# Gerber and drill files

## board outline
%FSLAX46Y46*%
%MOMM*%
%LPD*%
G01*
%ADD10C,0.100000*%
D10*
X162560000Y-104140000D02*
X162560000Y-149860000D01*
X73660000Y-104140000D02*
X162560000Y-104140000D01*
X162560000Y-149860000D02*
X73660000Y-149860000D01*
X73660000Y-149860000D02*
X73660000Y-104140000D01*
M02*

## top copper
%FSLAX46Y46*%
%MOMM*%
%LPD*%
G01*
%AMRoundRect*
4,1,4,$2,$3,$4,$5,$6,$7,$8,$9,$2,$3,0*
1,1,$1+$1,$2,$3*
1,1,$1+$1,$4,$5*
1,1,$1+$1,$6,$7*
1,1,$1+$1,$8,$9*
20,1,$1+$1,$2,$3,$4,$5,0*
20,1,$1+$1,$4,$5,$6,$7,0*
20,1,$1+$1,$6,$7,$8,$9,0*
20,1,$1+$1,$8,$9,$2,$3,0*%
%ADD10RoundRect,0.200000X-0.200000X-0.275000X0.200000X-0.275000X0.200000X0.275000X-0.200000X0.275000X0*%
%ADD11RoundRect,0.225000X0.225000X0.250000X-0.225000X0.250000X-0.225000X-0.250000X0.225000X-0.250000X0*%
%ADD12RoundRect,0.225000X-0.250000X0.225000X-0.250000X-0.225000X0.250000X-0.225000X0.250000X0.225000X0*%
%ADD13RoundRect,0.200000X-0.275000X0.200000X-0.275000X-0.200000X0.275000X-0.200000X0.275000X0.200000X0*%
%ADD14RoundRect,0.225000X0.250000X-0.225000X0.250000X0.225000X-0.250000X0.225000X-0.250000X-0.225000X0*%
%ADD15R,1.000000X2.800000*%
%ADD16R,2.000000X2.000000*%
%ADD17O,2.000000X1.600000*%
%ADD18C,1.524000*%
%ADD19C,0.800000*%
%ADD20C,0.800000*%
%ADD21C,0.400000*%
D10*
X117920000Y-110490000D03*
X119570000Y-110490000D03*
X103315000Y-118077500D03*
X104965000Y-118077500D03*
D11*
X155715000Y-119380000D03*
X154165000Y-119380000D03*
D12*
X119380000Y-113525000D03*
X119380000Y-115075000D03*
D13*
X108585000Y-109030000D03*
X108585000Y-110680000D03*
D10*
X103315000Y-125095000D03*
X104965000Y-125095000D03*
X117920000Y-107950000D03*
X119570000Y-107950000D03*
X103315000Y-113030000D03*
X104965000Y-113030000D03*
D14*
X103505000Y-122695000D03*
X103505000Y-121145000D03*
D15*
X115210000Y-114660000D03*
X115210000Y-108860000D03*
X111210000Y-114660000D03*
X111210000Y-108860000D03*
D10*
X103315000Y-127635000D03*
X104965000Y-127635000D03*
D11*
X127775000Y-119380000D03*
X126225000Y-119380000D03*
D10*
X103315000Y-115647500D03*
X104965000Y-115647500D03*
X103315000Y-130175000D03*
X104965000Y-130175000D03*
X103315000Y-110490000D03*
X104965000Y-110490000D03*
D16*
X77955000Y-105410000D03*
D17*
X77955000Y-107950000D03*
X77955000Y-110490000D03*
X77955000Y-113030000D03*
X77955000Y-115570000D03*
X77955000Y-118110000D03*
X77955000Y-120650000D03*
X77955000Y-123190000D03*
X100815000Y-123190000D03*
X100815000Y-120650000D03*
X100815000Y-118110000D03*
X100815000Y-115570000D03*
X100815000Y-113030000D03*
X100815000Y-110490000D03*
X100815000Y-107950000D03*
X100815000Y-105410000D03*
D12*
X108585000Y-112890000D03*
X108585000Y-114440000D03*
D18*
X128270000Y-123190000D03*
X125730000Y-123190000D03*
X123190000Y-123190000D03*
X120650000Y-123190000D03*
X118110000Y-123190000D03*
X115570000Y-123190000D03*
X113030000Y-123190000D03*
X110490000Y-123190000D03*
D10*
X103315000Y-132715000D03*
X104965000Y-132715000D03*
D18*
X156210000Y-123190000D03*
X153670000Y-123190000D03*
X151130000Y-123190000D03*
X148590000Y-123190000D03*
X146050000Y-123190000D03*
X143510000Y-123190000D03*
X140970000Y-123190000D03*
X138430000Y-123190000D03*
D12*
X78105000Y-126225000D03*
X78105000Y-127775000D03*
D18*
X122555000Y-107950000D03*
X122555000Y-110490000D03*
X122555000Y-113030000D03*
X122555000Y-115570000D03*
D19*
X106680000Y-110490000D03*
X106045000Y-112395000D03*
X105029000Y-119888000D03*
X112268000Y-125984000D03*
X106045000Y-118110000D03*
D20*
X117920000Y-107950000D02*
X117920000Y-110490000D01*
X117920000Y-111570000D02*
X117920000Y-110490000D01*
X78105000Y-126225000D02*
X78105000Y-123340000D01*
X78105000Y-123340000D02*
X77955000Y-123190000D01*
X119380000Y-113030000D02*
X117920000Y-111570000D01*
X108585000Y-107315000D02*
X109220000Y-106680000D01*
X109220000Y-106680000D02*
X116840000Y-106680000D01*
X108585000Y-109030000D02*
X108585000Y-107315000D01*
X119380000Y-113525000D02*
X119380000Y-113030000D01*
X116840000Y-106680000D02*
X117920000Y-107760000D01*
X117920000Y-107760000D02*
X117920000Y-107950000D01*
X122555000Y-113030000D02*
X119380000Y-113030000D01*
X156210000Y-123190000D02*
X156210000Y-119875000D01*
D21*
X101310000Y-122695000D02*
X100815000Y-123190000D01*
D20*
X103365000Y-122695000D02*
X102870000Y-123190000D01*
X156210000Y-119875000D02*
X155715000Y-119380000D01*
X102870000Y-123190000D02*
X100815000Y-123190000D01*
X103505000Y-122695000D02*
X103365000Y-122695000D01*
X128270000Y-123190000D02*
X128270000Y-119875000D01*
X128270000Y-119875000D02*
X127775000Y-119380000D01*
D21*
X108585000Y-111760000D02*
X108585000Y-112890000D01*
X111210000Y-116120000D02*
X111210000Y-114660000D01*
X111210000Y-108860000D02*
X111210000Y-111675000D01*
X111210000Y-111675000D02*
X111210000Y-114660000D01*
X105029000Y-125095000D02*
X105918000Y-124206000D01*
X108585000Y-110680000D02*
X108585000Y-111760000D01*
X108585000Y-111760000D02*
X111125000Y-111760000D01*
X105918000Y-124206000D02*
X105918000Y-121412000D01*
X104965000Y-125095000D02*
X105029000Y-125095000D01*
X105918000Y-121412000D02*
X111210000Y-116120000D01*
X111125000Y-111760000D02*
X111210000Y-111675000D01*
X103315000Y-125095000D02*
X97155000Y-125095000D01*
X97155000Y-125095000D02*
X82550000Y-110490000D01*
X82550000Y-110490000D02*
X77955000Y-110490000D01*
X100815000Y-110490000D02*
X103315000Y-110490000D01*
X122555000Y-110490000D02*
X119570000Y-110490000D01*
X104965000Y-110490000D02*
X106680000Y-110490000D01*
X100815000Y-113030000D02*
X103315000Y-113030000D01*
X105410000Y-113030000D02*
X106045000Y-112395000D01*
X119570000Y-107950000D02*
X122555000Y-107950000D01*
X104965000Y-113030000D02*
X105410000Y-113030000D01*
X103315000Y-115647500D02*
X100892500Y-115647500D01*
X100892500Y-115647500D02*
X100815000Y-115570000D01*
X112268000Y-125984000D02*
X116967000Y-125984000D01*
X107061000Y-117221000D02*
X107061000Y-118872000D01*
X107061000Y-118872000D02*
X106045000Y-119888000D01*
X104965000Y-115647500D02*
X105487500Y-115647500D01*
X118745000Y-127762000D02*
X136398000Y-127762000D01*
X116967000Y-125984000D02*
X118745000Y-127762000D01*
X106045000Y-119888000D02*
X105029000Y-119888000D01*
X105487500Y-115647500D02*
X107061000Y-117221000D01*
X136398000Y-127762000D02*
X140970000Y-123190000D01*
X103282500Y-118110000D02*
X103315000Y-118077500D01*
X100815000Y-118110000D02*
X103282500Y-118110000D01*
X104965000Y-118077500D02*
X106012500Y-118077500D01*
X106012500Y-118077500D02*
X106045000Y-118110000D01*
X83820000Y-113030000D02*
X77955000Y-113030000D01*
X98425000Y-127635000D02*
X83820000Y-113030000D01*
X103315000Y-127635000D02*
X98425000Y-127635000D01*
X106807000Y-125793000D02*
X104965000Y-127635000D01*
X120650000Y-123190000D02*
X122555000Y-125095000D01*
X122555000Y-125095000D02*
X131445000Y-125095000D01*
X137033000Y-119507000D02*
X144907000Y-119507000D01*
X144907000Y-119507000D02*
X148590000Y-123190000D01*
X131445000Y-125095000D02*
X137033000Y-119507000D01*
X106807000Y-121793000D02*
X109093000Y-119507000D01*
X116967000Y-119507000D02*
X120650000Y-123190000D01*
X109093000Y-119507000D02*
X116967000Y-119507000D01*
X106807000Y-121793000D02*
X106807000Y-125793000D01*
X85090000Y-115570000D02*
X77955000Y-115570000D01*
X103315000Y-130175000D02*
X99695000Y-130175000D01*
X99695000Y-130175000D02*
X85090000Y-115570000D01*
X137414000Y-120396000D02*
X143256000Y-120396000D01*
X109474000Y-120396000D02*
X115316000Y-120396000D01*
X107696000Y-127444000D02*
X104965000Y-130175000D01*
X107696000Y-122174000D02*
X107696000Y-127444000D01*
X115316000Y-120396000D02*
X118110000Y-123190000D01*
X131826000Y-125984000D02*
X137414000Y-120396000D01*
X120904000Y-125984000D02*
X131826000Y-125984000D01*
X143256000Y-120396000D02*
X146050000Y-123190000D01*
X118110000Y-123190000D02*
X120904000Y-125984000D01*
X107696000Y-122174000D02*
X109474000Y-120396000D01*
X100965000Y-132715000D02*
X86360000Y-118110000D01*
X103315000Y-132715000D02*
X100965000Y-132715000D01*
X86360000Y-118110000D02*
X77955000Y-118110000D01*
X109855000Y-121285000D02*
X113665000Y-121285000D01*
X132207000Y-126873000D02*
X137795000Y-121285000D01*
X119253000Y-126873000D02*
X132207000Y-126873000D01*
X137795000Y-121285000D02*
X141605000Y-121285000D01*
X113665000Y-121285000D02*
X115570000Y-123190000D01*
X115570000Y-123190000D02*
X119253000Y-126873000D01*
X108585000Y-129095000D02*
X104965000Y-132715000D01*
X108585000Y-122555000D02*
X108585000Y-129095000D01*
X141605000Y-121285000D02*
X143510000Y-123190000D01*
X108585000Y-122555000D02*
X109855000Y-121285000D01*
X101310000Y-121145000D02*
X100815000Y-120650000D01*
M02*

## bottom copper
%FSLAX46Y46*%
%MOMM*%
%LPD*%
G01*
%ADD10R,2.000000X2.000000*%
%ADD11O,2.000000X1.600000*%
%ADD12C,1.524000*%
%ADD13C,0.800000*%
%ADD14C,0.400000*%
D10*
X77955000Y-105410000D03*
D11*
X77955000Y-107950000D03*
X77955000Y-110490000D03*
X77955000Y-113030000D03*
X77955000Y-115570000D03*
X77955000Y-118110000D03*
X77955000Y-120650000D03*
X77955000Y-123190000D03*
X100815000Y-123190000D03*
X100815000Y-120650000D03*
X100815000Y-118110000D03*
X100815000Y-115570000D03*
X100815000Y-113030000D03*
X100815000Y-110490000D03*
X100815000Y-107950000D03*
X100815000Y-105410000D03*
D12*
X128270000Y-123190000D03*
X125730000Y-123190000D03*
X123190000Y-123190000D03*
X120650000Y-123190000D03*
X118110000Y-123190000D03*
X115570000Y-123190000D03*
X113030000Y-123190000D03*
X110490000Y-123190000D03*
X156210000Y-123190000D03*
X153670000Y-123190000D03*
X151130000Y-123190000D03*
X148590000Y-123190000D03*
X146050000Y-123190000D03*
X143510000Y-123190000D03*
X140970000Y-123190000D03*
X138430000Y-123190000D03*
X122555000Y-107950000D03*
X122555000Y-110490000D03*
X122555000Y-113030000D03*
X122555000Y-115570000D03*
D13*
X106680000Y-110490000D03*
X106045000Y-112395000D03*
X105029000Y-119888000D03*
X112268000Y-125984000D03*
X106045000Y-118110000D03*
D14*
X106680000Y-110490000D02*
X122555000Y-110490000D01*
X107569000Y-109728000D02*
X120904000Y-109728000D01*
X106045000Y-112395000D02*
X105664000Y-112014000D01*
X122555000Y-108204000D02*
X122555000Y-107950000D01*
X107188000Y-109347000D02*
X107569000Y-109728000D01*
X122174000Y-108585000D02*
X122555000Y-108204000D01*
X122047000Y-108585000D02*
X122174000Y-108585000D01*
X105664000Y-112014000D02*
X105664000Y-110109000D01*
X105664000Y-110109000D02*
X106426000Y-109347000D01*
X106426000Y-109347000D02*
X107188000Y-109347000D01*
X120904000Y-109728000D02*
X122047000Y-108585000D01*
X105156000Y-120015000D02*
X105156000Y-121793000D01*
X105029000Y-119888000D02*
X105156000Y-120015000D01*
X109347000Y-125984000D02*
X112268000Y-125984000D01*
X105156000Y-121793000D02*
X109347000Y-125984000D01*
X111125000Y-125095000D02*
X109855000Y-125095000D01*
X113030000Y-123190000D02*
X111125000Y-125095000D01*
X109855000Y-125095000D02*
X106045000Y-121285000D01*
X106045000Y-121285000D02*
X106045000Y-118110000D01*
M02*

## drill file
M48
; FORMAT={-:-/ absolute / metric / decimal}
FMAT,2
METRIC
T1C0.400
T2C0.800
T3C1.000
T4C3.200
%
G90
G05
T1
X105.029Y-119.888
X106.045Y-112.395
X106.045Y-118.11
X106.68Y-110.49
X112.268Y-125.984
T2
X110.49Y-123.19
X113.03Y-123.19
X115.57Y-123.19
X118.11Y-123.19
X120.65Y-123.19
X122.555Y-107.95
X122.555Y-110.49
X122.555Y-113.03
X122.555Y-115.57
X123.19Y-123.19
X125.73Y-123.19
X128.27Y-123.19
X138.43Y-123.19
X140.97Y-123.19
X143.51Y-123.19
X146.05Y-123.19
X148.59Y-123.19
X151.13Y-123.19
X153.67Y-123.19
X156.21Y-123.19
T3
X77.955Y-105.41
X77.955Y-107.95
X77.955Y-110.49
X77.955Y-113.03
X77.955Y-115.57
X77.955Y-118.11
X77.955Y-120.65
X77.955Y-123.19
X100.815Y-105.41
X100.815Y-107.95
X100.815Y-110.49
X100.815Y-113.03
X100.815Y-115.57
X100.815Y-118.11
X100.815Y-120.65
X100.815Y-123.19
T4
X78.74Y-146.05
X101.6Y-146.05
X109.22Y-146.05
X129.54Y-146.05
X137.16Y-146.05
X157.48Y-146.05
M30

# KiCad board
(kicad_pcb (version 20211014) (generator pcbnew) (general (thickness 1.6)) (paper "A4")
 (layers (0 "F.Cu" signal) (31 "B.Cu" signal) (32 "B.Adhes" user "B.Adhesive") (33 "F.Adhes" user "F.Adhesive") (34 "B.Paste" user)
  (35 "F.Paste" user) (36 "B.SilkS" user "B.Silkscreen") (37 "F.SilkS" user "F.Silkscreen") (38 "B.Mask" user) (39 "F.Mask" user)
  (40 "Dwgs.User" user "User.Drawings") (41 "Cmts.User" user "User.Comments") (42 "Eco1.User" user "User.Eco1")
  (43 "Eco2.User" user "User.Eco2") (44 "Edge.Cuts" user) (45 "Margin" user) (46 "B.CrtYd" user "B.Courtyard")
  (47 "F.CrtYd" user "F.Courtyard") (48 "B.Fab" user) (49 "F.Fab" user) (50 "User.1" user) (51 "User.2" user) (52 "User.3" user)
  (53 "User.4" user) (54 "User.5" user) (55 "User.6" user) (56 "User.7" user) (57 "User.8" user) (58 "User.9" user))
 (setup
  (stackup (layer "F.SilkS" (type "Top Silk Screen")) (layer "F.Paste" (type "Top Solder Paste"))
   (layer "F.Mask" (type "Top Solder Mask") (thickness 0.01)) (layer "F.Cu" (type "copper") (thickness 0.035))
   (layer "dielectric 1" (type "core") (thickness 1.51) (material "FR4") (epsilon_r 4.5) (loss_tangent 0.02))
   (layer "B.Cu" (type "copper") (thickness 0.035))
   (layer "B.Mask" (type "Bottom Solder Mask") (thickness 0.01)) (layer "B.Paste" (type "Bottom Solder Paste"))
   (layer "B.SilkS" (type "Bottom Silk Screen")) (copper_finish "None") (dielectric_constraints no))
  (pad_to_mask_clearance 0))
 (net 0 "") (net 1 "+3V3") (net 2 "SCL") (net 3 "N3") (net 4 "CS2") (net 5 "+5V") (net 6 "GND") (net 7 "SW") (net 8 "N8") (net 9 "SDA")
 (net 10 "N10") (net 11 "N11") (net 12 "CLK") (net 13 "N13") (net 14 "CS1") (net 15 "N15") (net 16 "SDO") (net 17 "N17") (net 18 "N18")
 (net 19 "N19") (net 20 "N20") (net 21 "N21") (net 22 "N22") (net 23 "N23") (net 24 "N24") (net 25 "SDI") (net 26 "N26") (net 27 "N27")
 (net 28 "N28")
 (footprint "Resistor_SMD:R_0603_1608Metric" (layer "F.Cu") (at 118.745 110.49)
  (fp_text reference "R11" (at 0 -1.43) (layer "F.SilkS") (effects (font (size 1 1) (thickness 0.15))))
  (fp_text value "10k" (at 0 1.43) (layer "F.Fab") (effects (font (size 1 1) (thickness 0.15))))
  (pad "1" smd roundrect (at -0.825 0) (size 0.8 0.95) (layers "F.Cu" "F.Paste" "F.Mask") (roundrect_rratio 0.25) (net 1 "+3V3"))
  (pad "2" smd roundrect (at 0.825 0) (size 0.8 0.95) (layers "F.Cu" "F.Paste" "F.Mask") (roundrect_rratio 0.25) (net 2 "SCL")))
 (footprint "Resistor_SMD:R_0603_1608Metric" (layer "F.Cu") (at 104.14 118.0775)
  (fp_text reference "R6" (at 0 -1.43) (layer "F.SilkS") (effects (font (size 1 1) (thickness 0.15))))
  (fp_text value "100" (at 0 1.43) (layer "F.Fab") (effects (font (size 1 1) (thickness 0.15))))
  (pad "1" smd roundrect (at -0.825 0) (size 0.8 0.95) (layers "F.Cu" "F.Paste" "F.Mask") (roundrect_rratio 0.25) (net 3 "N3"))
  (pad "2" smd roundrect (at 0.825 0) (size 0.8 0.95) (layers "F.Cu" "F.Paste" "F.Mask") (roundrect_rratio 0.25) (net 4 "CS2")))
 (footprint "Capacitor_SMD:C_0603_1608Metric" (layer "F.Cu") (at 154.94 119.38 180)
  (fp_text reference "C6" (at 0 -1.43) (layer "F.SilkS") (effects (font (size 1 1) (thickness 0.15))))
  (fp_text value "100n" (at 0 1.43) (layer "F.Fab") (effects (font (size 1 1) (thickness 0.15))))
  (pad "1" smd roundrect (at -0.775 0 180) (size 0.9 0.95) (layers "F.Cu" "F.Paste" "F.Mask") (roundrect_rratio 0.25) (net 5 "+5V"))
  (pad "2" smd roundrect (at 0.775 0 180) (size 0.9 0.95) (layers "F.Cu" "F.Paste" "F.Mask") (roundrect_rratio 0.25) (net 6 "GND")))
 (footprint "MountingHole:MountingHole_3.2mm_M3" (layer "F.Cu") (at 109.22 146.05)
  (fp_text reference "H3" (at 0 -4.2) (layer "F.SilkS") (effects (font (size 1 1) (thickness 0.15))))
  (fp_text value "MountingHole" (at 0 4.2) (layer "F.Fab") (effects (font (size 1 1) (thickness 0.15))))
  (pad "" np_thru_hole circle (at 0 0) (size 3.2 3.2) (drill 3.2) (layers *.Cu *.Mask)))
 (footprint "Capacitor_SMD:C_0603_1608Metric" (layer "F.Cu") (at 119.38 114.3 -90)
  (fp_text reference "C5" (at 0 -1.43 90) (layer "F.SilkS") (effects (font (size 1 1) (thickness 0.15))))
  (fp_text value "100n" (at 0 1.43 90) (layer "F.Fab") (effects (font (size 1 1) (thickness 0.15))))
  (pad "1" smd roundrect (at -0.775 0 270) (size 0.9 0.95) (layers "F.Cu" "F.Paste" "F.Mask") (roundrect_rratio 0.25) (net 1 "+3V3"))
  (pad "2" smd roundrect (at 0.775 0 270) (size 0.9 0.95) (layers "F.Cu" "F.Paste" "F.Mask") (roundrect_rratio 0.25) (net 6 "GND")))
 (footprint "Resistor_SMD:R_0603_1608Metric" (layer "F.Cu") (at 108.585 109.855 -90)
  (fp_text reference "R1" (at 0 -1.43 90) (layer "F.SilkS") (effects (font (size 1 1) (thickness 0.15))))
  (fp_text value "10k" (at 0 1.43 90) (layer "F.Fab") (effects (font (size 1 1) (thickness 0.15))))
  (pad "1" smd roundrect (at -0.825 0 270) (size 0.8 0.95) (layers "F.Cu" "F.Paste" "F.Mask") (roundrect_rratio 0.25) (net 1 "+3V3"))
  (pad "2" smd roundrect (at 0.825 0 270) (size 0.8 0.95) (layers "F.Cu" "F.Paste" "F.Mask") (roundrect_rratio 0.25) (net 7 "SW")))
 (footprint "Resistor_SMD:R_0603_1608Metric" (layer "F.Cu") (at 104.14 125.095)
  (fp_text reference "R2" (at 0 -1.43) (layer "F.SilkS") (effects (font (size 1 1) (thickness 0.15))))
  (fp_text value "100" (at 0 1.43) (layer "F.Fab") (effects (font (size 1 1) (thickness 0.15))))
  (pad "1" smd roundrect (at -0.825 0) (size 0.8 0.95) (layers "F.Cu" "F.Paste" "F.Mask") (roundrect_rratio 0.25) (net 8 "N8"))
  (pad "2" smd roundrect (at 0.825 0) (size 0.8 0.95) (layers "F.Cu" "F.Paste" "F.Mask") (roundrect_rratio 0.25) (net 7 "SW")))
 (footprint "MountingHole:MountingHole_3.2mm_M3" (layer "F.Cu") (at 78.74 146.05)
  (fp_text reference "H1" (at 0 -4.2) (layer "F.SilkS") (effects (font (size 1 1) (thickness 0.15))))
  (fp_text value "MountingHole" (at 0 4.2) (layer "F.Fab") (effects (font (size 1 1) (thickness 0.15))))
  (pad "" np_thru_hole circle (at 0 0) (size 3.2 3.2) (drill 3.2) (layers *.Cu *.Mask)))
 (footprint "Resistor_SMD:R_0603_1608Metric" (layer "F.Cu") (at 118.745 107.95)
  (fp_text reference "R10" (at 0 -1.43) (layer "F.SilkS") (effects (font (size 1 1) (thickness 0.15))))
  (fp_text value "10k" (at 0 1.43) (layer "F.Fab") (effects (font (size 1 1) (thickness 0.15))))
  (pad "1" smd roundrect (at -0.825 0) (size 0.8 0.95) (layers "F.Cu" "F.Paste" "F.Mask") (roundrect_rratio 0.25) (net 1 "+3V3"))
  (pad "2" smd roundrect (at 0.825 0) (size 0.8 0.95) (layers "F.Cu" "F.Paste" "F.Mask") (roundrect_rratio 0.25) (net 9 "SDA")))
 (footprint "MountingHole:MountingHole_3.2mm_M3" (layer "F.Cu") (at 137.16 146.05)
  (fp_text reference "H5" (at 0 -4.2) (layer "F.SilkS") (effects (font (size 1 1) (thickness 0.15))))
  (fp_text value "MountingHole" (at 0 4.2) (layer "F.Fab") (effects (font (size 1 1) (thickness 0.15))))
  (pad "" np_thru_hole circle (at 0 0) (size 3.2 3.2) (drill 3.2) (layers *.Cu *.Mask)))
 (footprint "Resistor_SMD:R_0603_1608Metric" (layer "F.Cu") (at 104.14 113.03)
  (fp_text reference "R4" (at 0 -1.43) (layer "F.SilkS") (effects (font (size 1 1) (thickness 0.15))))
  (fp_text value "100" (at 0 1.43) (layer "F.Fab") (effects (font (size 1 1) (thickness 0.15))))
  (pad "1" smd roundrect (at -0.825 0) (size 0.8 0.95) (layers "F.Cu" "F.Paste" "F.Mask") (roundrect_rratio 0.25) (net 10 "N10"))
  (pad "2" smd roundrect (at 0.825 0) (size 0.8 0.95) (layers "F.Cu" "F.Paste" "F.Mask") (roundrect_rratio 0.25) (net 9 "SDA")))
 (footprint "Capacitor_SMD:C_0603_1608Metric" (layer "F.Cu") (at 103.505 121.92 90)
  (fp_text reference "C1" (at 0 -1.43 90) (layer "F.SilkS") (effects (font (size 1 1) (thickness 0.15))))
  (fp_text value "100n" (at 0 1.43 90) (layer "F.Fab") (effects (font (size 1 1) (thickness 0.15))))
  (pad "1" smd roundrect (at -0.775 0 90) (size 0.9 0.95) (layers "F.Cu" "F.Paste" "F.Mask") (roundrect_rratio 0.25) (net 5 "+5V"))
  (pad "2" smd roundrect (at 0.775 0 90) (size 0.9 0.95) (layers "F.Cu" "F.Paste" "F.Mask") (roundrect_rratio 0.25) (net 6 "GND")))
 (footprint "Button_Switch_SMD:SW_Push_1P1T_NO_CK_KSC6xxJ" (layer "F.Cu") (at 113.21 111.76 -90)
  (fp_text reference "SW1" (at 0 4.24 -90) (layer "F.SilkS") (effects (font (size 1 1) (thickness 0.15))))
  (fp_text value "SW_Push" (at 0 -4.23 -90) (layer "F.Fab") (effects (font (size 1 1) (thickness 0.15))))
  (pad "1" smd rect (at 2.9 -2 270) (size 2.8 1) (layers "F.Cu" "F.Paste" "F.Mask") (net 6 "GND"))
  (pad "1" smd rect (at -2.9 -2 270) (size 2.8 1) (layers "F.Cu" "F.Paste" "F.Mask") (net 6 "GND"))
  (pad "2" smd rect (at 2.9 2 270) (size 2.8 1) (layers "F.Cu" "F.Paste" "F.Mask") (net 7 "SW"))
  (pad "2" smd rect (at -2.9 2 270) (size 2.8 1) (layers "F.Cu" "F.Paste" "F.Mask") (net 7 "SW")))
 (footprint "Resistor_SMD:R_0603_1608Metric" (layer "F.Cu") (at 104.14 127.635)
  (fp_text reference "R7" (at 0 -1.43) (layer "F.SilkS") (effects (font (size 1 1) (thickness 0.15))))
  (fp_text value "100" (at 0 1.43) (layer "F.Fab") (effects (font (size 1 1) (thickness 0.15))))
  (pad "1" smd roundrect (at -0.825 0) (size 0.8 0.95) (layers "F.Cu" "F.Paste" "F.Mask") (roundrect_rratio 0.25) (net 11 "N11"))
  (pad "2" smd roundrect (at 0.825 0) (size 0.8 0.95) (layers "F.Cu" "F.Paste" "F.Mask") (roundrect_rratio 0.25) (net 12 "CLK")))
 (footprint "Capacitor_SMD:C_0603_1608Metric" (layer "F.Cu") (at 127 119.38 180)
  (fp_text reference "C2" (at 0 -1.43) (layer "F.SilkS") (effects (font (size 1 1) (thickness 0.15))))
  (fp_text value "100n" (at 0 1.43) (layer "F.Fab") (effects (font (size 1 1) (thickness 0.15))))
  (pad "1" smd roundrect (at -0.775 0 180) (size 0.9 0.95) (layers "F.Cu" "F.Paste" "F.Mask") (roundrect_rratio 0.25) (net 5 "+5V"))
  (pad "2" smd roundrect (at 0.775 0 180) (size 0.9 0.95) (layers "F.Cu" "F.Paste" "F.Mask") (roundrect_rratio 0.25) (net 6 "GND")))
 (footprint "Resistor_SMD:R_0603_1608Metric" (layer "F.Cu") (at 104.14 115.6475)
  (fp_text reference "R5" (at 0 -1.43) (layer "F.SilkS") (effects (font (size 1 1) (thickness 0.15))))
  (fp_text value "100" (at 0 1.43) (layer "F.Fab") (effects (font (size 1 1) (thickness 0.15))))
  (pad "1" smd roundrect (at -0.825 0) (size 0.8 0.95) (layers "F.Cu" "F.Paste" "F.Mask") (roundrect_rratio 0.25) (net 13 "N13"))
  (pad "2" smd roundrect (at 0.825 0) (size 0.8 0.95) (layers "F.Cu" "F.Paste" "F.Mask") (roundrect_rratio 0.25) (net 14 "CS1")))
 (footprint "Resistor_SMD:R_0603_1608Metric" (layer "F.Cu") (at 104.14 130.175)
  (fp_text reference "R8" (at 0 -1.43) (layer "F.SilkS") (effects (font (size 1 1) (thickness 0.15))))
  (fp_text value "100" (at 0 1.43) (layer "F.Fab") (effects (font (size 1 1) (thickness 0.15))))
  (pad "1" smd roundrect (at -0.825 0) (size 0.8 0.95) (layers "F.Cu" "F.Paste" "F.Mask") (roundrect_rratio 0.25) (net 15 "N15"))
  (pad "2" smd roundrect (at 0.825 0) (size 0.8 0.95) (layers "F.Cu" "F.Paste" "F.Mask") (roundrect_rratio 0.25) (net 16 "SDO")))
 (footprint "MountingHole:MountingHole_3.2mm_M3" (layer "F.Cu") (at 157.479999 146.049999)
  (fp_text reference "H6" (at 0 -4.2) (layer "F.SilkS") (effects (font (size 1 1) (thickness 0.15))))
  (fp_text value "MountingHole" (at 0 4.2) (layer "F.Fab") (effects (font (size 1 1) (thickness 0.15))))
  (pad "" np_thru_hole circle (at 0 0) (size 3.2 3.2) (drill 3.2) (layers *.Cu *.Mask)))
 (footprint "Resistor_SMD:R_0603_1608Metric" (layer "F.Cu") (at 104.14 110.49)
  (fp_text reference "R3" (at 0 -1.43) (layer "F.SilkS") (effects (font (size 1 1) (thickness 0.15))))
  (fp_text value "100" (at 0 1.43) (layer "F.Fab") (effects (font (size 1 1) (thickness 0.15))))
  (pad "1" smd roundrect (at -0.825 0) (size 0.8 0.95) (layers "F.Cu" "F.Paste" "F.Mask") (roundrect_rratio 0.25) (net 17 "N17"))
  (pad "2" smd roundrect (at 0.825 0) (size 0.8 0.95) (layers "F.Cu" "F.Paste" "F.Mask") (roundrect_rratio 0.25) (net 2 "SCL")))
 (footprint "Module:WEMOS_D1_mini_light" (layer "F.Cu") (at 77.955 105.41)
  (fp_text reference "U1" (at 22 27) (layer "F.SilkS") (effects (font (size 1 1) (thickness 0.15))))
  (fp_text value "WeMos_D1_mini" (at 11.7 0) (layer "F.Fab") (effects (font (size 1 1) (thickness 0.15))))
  (pad "1" thru_hole rect (at 0 0) (size 2 2) (drill 1) (layers *.Cu *.Mask) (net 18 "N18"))
  (pad "2" thru_hole oval (at 0 2.54) (size 2 1.6) (drill 1) (layers *.Cu *.Mask) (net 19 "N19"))
  (pad "3" thru_hole oval (at 0 5.08) (size 2 1.6) (drill 1) (layers *.Cu *.Mask) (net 8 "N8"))
  (pad "4" thru_hole oval (at 0 7.62) (size 2 1.6) (drill 1) (layers *.Cu *.Mask) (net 11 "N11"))
  (pad "5" thru_hole oval (at 0 10.16) (size 2 1.6) (drill 1) (layers *.Cu *.Mask) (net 15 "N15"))
  (pad "6" thru_hole oval (at 0 12.7) (size 2 1.6) (drill 1) (layers *.Cu *.Mask) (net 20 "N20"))
  (pad "7" thru_hole oval (at 0 15.24) (size 2 1.6) (drill 1) (layers *.Cu *.Mask) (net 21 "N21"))
  (pad "8" thru_hole oval (at 0 17.78) (size 2 1.6) (drill 1) (layers *.Cu *.Mask) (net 1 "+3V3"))
  (pad "9" thru_hole oval (at 22.86 17.78) (size 2 1.6) (drill 1) (layers *.Cu *.Mask) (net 5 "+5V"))
  (pad "10" thru_hole oval (at 22.86 15.24) (size 2 1.6) (drill 1) (layers *.Cu *.Mask) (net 6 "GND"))
  (pad "11" thru_hole oval (at 22.86 12.7) (size 2 1.6) (drill 1) (layers *.Cu *.Mask) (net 3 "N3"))
  (pad "12" thru_hole oval (at 22.86 10.16) (size 2 1.6) (drill 1) (layers *.Cu *.Mask) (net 13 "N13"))
  (pad "13" thru_hole oval (at 22.86 7.62) (size 2 1.6) (drill 1) (layers *.Cu *.Mask) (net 10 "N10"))
  (pad "14" thru_hole oval (at 22.86 5.08) (size 2 1.6) (drill 1) (layers *.Cu *.Mask) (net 17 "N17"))
  (pad "15" thru_hole oval (at 22.86 2.54) (size 2 1.6) (drill 1) (layers *.Cu *.Mask) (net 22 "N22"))
  (pad "16" thru_hole oval (at 22.86 0) (size 2 1.6) (drill 1) (layers *.Cu *.Mask) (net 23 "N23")))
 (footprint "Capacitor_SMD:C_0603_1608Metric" (layer "F.Cu") (at 108.585 113.665 -90)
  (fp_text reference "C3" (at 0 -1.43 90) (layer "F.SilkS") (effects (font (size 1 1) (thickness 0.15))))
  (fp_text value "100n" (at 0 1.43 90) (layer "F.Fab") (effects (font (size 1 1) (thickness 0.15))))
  (pad "1" smd roundrect (at -0.775 0 270) (size 0.9 0.95) (layers "F.Cu" "F.Paste" "F.Mask") (roundrect_rratio 0.25) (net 7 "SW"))
  (pad "2" smd roundrect (at 0.775 0 270) (size 0.9 0.95) (layers "F.Cu" "F.Paste" "F.Mask") (roundrect_rratio 0.25) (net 6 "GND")))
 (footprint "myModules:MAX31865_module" (layer "F.Cu") (at 118.11 128.27 180)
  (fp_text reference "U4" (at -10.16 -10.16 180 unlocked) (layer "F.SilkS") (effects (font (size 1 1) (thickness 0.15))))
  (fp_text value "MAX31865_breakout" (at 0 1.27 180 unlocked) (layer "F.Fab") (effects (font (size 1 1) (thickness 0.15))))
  (pad "1" thru_hole circle (at -10.16 5.08 180) (size 1.524 1.524) (drill 0.8) (layers *.Cu *.Mask) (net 5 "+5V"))
  (pad "2" thru_hole circle (at -7.62 5.08 180) (size 1.524 1.524) (drill 0.8) (layers *.Cu *.Mask) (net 6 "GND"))
  (pad "3" thru_hole circle (at -5.08 5.08 180) (size 1.524 1.524) (drill 0.8) (layers *.Cu *.Mask) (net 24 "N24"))
  (pad "4" thru_hole circle (at -2.54 5.08 180) (size 1.524 1.524) (drill 0.8) (layers *.Cu *.Mask) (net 12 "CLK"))
  (pad "5" thru_hole circle (at 0 5.08 180) (size 1.524 1.524) (drill 0.8) (layers *.Cu *.Mask) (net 16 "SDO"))
  (pad "6" thru_hole circle (at 2.54 5.08 180) (size 1.524 1.524) (drill 0.8) (layers *.Cu *.Mask) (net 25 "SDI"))
  (pad "7" thru_hole circle (at 5.08 5.08 180) (size 1.524 1.524) (drill 0.8) (layers *.Cu *.Mask) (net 4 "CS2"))
  (pad "8" thru_hole circle (at 7.62 5.08 180) (size 1.524 1.524) (drill 0.8) (layers *.Cu *.Mask) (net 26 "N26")))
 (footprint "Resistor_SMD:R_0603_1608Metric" (layer "F.Cu") (at 104.14 132.715)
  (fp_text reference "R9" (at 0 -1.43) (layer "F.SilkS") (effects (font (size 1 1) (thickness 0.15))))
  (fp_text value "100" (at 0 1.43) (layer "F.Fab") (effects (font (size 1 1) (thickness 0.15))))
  (pad "1" smd roundrect (at -0.825 0) (size 0.8 0.95) (layers "F.Cu" "F.Paste" "F.Mask") (roundrect_rratio 0.25) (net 20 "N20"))
  (pad "2" smd roundrect (at 0.825 0) (size 0.8 0.95) (layers "F.Cu" "F.Paste" "F.Mask") (roundrect_rratio 0.25) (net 25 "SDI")))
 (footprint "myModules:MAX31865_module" (layer "F.Cu") (at 146.05 128.27 180)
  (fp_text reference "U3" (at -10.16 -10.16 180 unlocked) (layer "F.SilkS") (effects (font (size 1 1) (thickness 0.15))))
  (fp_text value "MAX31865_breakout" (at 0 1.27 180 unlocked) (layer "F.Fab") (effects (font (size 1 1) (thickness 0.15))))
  (pad "1" thru_hole circle (at -10.16 5.08 180) (size 1.524 1.524) (drill 0.8) (layers *.Cu *.Mask) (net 5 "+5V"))
  (pad "2" thru_hole circle (at -7.62 5.08 180) (size 1.524 1.524) (drill 0.8) (layers *.Cu *.Mask) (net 6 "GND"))
  (pad "3" thru_hole circle (at -5.08 5.08 180) (size 1.524 1.524) (drill 0.8) (layers *.Cu *.Mask) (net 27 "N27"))
  (pad "4" thru_hole circle (at -2.54 5.08 180) (size 1.524 1.524) (drill 0.8) (layers *.Cu *.Mask) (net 12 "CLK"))
  (pad "5" thru_hole circle (at 0 5.08 180) (size 1.524 1.524) (drill 0.8) (layers *.Cu *.Mask) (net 16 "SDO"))
  (pad "6" thru_hole circle (at 2.54 5.08 180) (size 1.524 1.524) (drill 0.8) (layers *.Cu *.Mask) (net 25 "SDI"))
  (pad "7" thru_hole circle (at 5.08 5.08 180) (size 1.524 1.524) (drill 0.8) (layers *.Cu *.Mask) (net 14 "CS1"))
  (pad "8" thru_hole circle (at 7.62 5.08 180) (size 1.524 1.524) (drill 0.8) (layers *.Cu *.Mask) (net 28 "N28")))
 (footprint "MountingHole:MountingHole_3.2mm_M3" (layer "F.Cu") (at 101.6 146.05)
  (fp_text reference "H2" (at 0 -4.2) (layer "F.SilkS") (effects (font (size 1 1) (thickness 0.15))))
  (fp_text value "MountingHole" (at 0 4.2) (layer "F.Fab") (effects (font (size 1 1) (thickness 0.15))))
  (pad "" np_thru_hole circle (at 0 0) (size 3.2 3.2) (drill 3.2) (layers *.Cu *.Mask)))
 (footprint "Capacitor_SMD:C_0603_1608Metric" (layer "F.Cu") (at 78.105 127 -90)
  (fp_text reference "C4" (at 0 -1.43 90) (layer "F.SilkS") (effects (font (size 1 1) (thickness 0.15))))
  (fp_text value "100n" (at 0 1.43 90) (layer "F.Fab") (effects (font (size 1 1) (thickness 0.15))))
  (pad "1" smd roundrect (at -0.775 0 270) (size 0.9 0.95) (layers "F.Cu" "F.Paste" "F.Mask") (roundrect_rratio 0.25) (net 1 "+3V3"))
  (pad "2" smd roundrect (at 0.775 0 270) (size 0.9 0.95) (layers "F.Cu" "F.Paste" "F.Mask") (roundrect_rratio 0.25) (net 6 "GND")))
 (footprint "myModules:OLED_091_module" (layer "F.Cu") (at 122.555 111.76)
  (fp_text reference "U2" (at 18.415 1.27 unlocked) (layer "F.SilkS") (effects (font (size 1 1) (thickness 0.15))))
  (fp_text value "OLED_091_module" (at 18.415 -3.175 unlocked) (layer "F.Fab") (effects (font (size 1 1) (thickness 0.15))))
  (pad "1" thru_hole circle (at 0 -3.81) (size 1.524 1.524) (drill 0.8) (layers *.Cu *.Mask) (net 9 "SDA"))
  (pad "2" thru_hole circle (at 0 -1.27) (size 1.524 1.524) (drill 0.8) (layers *.Cu *.Mask) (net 2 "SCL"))
  (pad "3" thru_hole circle (at 0 1.27) (size 1.524 1.524) (drill 0.8) (layers *.Cu *.Mask) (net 1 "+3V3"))
  (pad "4" thru_hole circle (at 0 3.81) (size 1.524 1.524) (drill 0.8) (layers *.Cu *.Mask) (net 6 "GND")))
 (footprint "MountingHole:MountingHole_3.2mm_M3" (layer "F.Cu") (at 129.54 146.05)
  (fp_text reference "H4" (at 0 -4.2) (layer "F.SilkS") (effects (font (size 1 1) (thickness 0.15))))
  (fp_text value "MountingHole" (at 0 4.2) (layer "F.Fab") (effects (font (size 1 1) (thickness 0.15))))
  (pad "" np_thru_hole circle (at 0 0) (size 3.2 3.2) (drill 3.2) (layers *.Cu *.Mask)))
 (gr_line (start 162.56 104.14) (end 162.56 149.86) (layer "Edge.Cuts") (width 0.1))
 (gr_line (start 73.66 104.14) (end 162.56 104.14) (layer "Edge.Cuts") (width 0.1))
 (gr_line (start 162.56 149.86) (end 73.66 149.86) (layer "Edge.Cuts") (width 0.1))
 (gr_line (start 73.66 149.86) (end 73.66 104.14) (layer "Edge.Cuts") (width 0.1))
 (segment (start 117.92 107.95) (end 117.92 110.49) (width 0.8) (layer "F.Cu") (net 1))
 (segment (start 117.92 111.57) (end 117.92 110.49) (width 0.8) (layer "F.Cu") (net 1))
 (segment (start 78.105 126.225) (end 78.105 123.34) (width 0.8) (layer "F.Cu") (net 1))
 (segment (start 78.105 123.34) (end 77.955 123.19) (width 0.8) (layer "F.Cu") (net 1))
 (segment (start 119.38 113.03) (end 117.92 111.57) (width 0.8) (layer "F.Cu") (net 1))
 (segment (start 108.585 107.315) (end 109.22 106.68) (width 0.8) (layer "F.Cu") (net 1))
 (segment (start 109.22 106.68) (end 116.84 106.68) (width 0.8) (layer "F.Cu") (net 1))
 (segment (start 108.585 109.03) (end 108.585 107.315) (width 0.8) (layer "F.Cu") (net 1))
 (segment (start 119.38 113.525) (end 119.38 113.03) (width 0.8) (layer "F.Cu") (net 1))
 (segment (start 116.84 106.68) (end 117.92 107.76) (width 0.8) (layer "F.Cu") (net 1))
 (segment (start 117.92 107.76) (end 117.92 107.95) (width 0.8) (layer "F.Cu") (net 1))
 (segment (start 122.555 113.03) (end 119.38 113.03) (width 0.8) (layer "F.Cu") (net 1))
 (segment (start 156.21 123.19) (end 156.21 119.875) (width 0.8) (layer "F.Cu") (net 5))
 (segment (start 101.31 122.695) (end 100.815 123.19) (width 0.4) (layer "F.Cu") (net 5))
 (segment (start 103.365 122.695) (end 102.87 123.19) (width 0.8) (layer "F.Cu") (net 5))
 (segment (start 156.21 119.875) (end 155.715 119.38) (width 0.8) (layer "F.Cu") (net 5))
 (segment (start 102.87 123.19) (end 100.815 123.19) (width 0.8) (layer "F.Cu") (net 5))
 (segment (start 103.505 122.695) (end 103.365 122.695) (width 0.8) (layer "F.Cu") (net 5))
 (segment (start 128.27 123.19) (end 128.27 119.875) (width 0.8) (layer "F.Cu") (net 5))
 (segment (start 128.27 119.875) (end 127.775 119.38) (width 0.8) (layer "F.Cu") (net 5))
 (segment (start 108.585 111.76) (end 108.585 112.89) (width 0.4) (layer "F.Cu") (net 7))
 (segment (start 111.21 116.12) (end 111.21 114.66) (width 0.4) (layer "F.Cu") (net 7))
 (segment (start 111.21 108.86) (end 111.21 111.675) (width 0.4) (layer "F.Cu") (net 7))
 (segment (start 111.21 111.675) (end 111.21 114.66) (width 0.4) (layer "F.Cu") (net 7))
 (segment (start 105.029 125.095) (end 105.918 124.206) (width 0.4) (layer "F.Cu") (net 7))
 (segment (start 108.585 110.68) (end 108.585 111.76) (width 0.4) (layer "F.Cu") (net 7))
 (segment (start 108.585 111.76) (end 111.125 111.76) (width 0.4) (layer "F.Cu") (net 7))
 (segment (start 105.918 124.206) (end 105.918 121.412) (width 0.4) (layer "F.Cu") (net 7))
 (segment (start 104.965 125.095) (end 105.029 125.095) (width 0.4) (layer "F.Cu") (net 7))
 (segment (start 105.918 121.412) (end 111.21 116.12) (width 0.4) (layer "F.Cu") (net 7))
 (segment (start 111.125 111.76) (end 111.21 111.675) (width 0.4) (layer "F.Cu") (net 7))
 (segment (start 103.315 125.095) (end 97.155 125.095) (width 0.4) (layer "F.Cu") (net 8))
 (segment (start 97.155 125.095) (end 82.55 110.49) (width 0.4) (layer "F.Cu") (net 8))
 (segment (start 82.55 110.49) (end 77.955 110.49) (width 0.4) (layer "F.Cu") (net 8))
 (segment (start 100.815 110.49) (end 103.315 110.49) (width 0.4) (layer "F.Cu") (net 17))
 (segment (start 122.555 110.49) (end 119.57 110.49) (width 0.4) (layer "F.Cu") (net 2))
 (segment (start 104.965 110.49) (end 106.68 110.49) (width 0.4) (layer "F.Cu") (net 2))
 (via (at 106.68 110.49) (size 0.8) (drill 0.4) (layers "F.Cu" "B.Cu") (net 2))
 (segment (start 106.68 110.49) (end 122.555 110.49) (width 0.4) (layer "B.Cu") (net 2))
 (segment (start 100.815 113.03) (end 103.315 113.03) (width 0.4) (layer "F.Cu") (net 10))
 (segment (start 105.41 113.03) (end 106.045 112.395) (width 0.4) (layer "F.Cu") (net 9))
 (segment (start 119.57 107.95) (end 122.555 107.95) (width 0.4) (layer "F.Cu") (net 9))
 (segment (start 104.965 113.03) (end 105.41 113.03) (width 0.4) (layer "F.Cu") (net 9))
 (via (at 106.045 112.395) (size 0.8) (drill 0.4) (layers "F.Cu" "B.Cu") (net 9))
 (segment (start 107.569 109.728) (end 120.904 109.728) (width 0.4) (layer "B.Cu") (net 9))
 (segment (start 106.045 112.395) (end 105.664 112.014) (width 0.4) (layer "B.Cu") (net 9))
 (segment (start 122.555 108.204) (end 122.555 107.95) (width 0.4) (layer "B.Cu") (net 9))
 (segment (start 107.188 109.347) (end 107.569 109.728) (width 0.4) (layer "B.Cu") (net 9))
 (segment (start 122.174 108.585) (end 122.555 108.204) (width 0.4) (layer "B.Cu") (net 9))
 (segment (start 122.047 108.585) (end 122.174 108.585) (width 0.4) (layer "B.Cu") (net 9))
 (segment (start 105.664 112.014) (end 105.664 110.109) (width 0.4) (layer "B.Cu") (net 9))
 (segment (start 105.664 110.109) (end 106.426 109.347) (width 0.4) (layer "B.Cu") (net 9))
 (segment (start 106.426 109.347) (end 107.188 109.347) (width 0.4) (layer "B.Cu") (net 9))
 (segment (start 120.904 109.728) (end 122.047 108.585) (width 0.4) (layer "B.Cu") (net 9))
 (segment (start 103.315 115.6475) (end 100.8925 115.6475) (width 0.4) (layer "F.Cu") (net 13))
 (segment (start 100.8925 115.6475) (end 100.815 115.57) (width 0.4) (layer "F.Cu") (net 13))
 (segment (start 112.268 125.984) (end 116.967 125.984) (width 0.4) (layer "F.Cu") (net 14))
 (segment (start 107.061 117.221) (end 107.061 118.872) (width 0.4) (layer "F.Cu") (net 14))
 (segment (start 107.061 118.872) (end 106.045 119.888) (width 0.4) (layer "F.Cu") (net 14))
 (segment (start 104.965 115.6475) (end 105.4875 115.6475) (width 0.4) (layer "F.Cu") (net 14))
 (segment (start 118.745 127.762) (end 136.398 127.762) (width 0.4) (layer "F.Cu") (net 14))
 (segment (start 116.967 125.984) (end 118.745 127.762) (width 0.4) (layer "F.Cu") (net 14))
 (segment (start 106.045 119.888) (end 105.029 119.888) (width 0.4) (layer "F.Cu") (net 14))
 (segment (start 105.4875 115.6475) (end 107.061 117.221) (width 0.4) (layer "F.Cu") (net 14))
 (segment (start 136.398 127.762) (end 140.97 123.19) (width 0.4) (layer "F.Cu") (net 14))
 (via (at 105.029 119.888) (size 0.8) (drill 0.4) (layers "F.Cu" "B.Cu") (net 14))
 (via (at 112.268 125.984) (size 0.8) (drill 0.4) (layers "F.Cu" "B.Cu") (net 14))
 (segment (start 105.156 120.015) (end 105.156 121.793) (width 0.4) (layer "B.Cu") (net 14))
 (segment (start 105.029 119.888) (end 105.156 120.015) (width 0.4) (layer "B.Cu") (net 14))
 (segment (start 109.347 125.984) (end 112.268 125.984) (width 0.4) (layer "B.Cu") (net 14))
 (segment (start 105.156 121.793) (end 109.347 125.984) (width 0.4) (layer "B.Cu") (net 14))
 (segment (start 103.2825 118.11) (end 103.315 118.0775) (width 0.4) (layer "F.Cu") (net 3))
 (segment (start 100.815 118.11) (end 103.2825 118.11) (width 0.4) (layer "F.Cu") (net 3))
 (segment (start 104.965 118.0775) (end 106.0125 118.0775) (width 0.4) (layer "F.Cu") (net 4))
 (segment (start 106.0125 118.0775) (end 106.045 118.11) (width 0.4) (layer "F.Cu") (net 4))
 (via (at 106.045 118.11) (size 0.8) (drill 0.4) (layers "F.Cu" "B.Cu") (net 4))
 (segment (start 111.125 125.095) (end 109.855 125.095) (width 0.4) (layer "B.Cu") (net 4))
 (segment (start 113.03 123.19) (end 111.125 125.095) (width 0.4) (layer "B.Cu") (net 4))
 (segment (start 109.855 125.095) (end 106.045 121.285) (width 0.4) (layer "B.Cu") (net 4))
 (segment (start 106.045 121.285) (end 106.045 118.11) (width 0.4) (layer "B.Cu") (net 4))
 (segment (start 83.82 113.03) (end 77.955 113.03) (width 0.4) (layer "F.Cu") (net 11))
 (segment (start 98.425 127.635) (end 83.82 113.03) (width 0.4) (layer "F.Cu") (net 11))
 (segment (start 103.315 127.635) (end 98.425 127.635) (width 0.4) (layer "F.Cu") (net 11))
 (segment (start 106.807 125.793) (end 104.965 127.635) (width 0.4) (layer "F.Cu") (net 12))
 (segment (start 120.65 123.19) (end 122.555 125.095) (width 0.4) (layer "F.Cu") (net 12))
 (segment (start 122.555 125.095) (end 131.445 125.095) (width 0.4) (layer "F.Cu") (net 12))
 (segment (start 137.033 119.507) (end 144.907 119.507) (width 0.4) (layer "F.Cu") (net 12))
 (segment (start 144.907 119.507) (end 148.59 123.19) (width 0.4) (layer "F.Cu") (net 12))
 (segment (start 131.445 125.095) (end 137.033 119.507) (width 0.4) (layer "F.Cu") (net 12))
 (segment (start 106.807 121.793) (end 109.093 119.507) (width 0.4) (layer "F.Cu") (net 12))
 (segment (start 116.967 119.507) (end 120.65 123.19) (width 0.4) (layer "F.Cu") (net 12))
 (segment (start 109.093 119.507) (end 116.967 119.507) (width 0.4) (layer "F.Cu") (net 12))
 (segment (start 106.807 121.793) (end 106.807 125.793) (width 0.4) (layer "F.Cu") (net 12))
 (segment (start 85.09 115.57) (end 77.955 115.57) (width 0.4) (layer "F.Cu") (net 15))
 (segment (start 103.315 130.175) (end 99.695 130.175) (width 0.4) (layer "F.Cu") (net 15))
 (segment (start 99.695 130.175) (end 85.09 115.57) (width 0.4) (layer "F.Cu") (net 15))
 (segment (start 137.414 120.396) (end 143.256 120.396) (width 0.4) (layer "F.Cu") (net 16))
 (segment (start 109.474 120.396) (end 115.316 120.396) (width 0.4) (layer "F.Cu") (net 16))
 (segment (start 107.696 127.444) (end 104.965 130.175) (width 0.4) (layer "F.Cu") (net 16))
 (segment (start 107.696 122.174) (end 107.696 127.444) (width 0.4) (layer "F.Cu") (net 16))
 (segment (start 115.316 120.396) (end 118.11 123.19) (width 0.4) (layer "F.Cu") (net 16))
 (segment (start 131.826 125.984) (end 137.414 120.396) (width 0.4) (layer "F.Cu") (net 16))
 (segment (start 120.904 125.984) (end 131.826 125.984) (width 0.4) (layer "F.Cu") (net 16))
 (segment (start 143.256 120.396) (end 146.05 123.19) (width 0.4) (layer "F.Cu") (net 16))
 (segment (start 118.11 123.19) (end 120.904 125.984) (width 0.4) (layer "F.Cu") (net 16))
 (segment (start 107.696 122.174) (end 109.474 120.396) (width 0.4) (layer "F.Cu") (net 16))
 (segment (start 100.965 132.715) (end 86.36 118.11) (width 0.4) (layer "F.Cu") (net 20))
 (segment (start 103.315 132.715) (end 100.965 132.715) (width 0.4) (layer "F.Cu") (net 20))
 (segment (start 86.36 118.11) (end 77.955 118.11) (width 0.4) (layer "F.Cu") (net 20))
 (segment (start 109.855 121.285) (end 113.665 121.285) (width 0.4) (layer "F.Cu") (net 25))
 (segment (start 132.207 126.873) (end 137.795 121.285) (width 0.4) (layer "F.Cu") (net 25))
 (segment (start 119.253 126.873) (end 132.207 126.873) (width 0.4) (layer "F.Cu") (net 25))
 (segment (start 137.795 121.285) (end 141.605 121.285) (width 0.4) (layer "F.Cu") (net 25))
 (segment (start 113.665 121.285) (end 115.57 123.19) (width 0.4) (layer "F.Cu") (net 25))
 (segment (start 115.57 123.19) (end 119.253 126.873) (width 0.4) (layer "F.Cu") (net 25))
 (segment (start 108.585 129.095) (end 104.965 132.715) (width 0.4) (layer "F.Cu") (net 25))
 (segment (start 108.585 122.555) (end 108.585 129.095) (width 0.4) (layer "F.Cu") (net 25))
 (segment (start 141.605 121.285) (end 143.51 123.19) (width 0.4) (layer "F.Cu") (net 25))
 (segment (start 108.585 122.555) (end 109.855 121.285) (width 0.4) (layer "F.Cu") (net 25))
 (segment (start 101.31 121.145) (end 100.815 120.65) (width 0.4) (layer "F.Cu") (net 6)))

